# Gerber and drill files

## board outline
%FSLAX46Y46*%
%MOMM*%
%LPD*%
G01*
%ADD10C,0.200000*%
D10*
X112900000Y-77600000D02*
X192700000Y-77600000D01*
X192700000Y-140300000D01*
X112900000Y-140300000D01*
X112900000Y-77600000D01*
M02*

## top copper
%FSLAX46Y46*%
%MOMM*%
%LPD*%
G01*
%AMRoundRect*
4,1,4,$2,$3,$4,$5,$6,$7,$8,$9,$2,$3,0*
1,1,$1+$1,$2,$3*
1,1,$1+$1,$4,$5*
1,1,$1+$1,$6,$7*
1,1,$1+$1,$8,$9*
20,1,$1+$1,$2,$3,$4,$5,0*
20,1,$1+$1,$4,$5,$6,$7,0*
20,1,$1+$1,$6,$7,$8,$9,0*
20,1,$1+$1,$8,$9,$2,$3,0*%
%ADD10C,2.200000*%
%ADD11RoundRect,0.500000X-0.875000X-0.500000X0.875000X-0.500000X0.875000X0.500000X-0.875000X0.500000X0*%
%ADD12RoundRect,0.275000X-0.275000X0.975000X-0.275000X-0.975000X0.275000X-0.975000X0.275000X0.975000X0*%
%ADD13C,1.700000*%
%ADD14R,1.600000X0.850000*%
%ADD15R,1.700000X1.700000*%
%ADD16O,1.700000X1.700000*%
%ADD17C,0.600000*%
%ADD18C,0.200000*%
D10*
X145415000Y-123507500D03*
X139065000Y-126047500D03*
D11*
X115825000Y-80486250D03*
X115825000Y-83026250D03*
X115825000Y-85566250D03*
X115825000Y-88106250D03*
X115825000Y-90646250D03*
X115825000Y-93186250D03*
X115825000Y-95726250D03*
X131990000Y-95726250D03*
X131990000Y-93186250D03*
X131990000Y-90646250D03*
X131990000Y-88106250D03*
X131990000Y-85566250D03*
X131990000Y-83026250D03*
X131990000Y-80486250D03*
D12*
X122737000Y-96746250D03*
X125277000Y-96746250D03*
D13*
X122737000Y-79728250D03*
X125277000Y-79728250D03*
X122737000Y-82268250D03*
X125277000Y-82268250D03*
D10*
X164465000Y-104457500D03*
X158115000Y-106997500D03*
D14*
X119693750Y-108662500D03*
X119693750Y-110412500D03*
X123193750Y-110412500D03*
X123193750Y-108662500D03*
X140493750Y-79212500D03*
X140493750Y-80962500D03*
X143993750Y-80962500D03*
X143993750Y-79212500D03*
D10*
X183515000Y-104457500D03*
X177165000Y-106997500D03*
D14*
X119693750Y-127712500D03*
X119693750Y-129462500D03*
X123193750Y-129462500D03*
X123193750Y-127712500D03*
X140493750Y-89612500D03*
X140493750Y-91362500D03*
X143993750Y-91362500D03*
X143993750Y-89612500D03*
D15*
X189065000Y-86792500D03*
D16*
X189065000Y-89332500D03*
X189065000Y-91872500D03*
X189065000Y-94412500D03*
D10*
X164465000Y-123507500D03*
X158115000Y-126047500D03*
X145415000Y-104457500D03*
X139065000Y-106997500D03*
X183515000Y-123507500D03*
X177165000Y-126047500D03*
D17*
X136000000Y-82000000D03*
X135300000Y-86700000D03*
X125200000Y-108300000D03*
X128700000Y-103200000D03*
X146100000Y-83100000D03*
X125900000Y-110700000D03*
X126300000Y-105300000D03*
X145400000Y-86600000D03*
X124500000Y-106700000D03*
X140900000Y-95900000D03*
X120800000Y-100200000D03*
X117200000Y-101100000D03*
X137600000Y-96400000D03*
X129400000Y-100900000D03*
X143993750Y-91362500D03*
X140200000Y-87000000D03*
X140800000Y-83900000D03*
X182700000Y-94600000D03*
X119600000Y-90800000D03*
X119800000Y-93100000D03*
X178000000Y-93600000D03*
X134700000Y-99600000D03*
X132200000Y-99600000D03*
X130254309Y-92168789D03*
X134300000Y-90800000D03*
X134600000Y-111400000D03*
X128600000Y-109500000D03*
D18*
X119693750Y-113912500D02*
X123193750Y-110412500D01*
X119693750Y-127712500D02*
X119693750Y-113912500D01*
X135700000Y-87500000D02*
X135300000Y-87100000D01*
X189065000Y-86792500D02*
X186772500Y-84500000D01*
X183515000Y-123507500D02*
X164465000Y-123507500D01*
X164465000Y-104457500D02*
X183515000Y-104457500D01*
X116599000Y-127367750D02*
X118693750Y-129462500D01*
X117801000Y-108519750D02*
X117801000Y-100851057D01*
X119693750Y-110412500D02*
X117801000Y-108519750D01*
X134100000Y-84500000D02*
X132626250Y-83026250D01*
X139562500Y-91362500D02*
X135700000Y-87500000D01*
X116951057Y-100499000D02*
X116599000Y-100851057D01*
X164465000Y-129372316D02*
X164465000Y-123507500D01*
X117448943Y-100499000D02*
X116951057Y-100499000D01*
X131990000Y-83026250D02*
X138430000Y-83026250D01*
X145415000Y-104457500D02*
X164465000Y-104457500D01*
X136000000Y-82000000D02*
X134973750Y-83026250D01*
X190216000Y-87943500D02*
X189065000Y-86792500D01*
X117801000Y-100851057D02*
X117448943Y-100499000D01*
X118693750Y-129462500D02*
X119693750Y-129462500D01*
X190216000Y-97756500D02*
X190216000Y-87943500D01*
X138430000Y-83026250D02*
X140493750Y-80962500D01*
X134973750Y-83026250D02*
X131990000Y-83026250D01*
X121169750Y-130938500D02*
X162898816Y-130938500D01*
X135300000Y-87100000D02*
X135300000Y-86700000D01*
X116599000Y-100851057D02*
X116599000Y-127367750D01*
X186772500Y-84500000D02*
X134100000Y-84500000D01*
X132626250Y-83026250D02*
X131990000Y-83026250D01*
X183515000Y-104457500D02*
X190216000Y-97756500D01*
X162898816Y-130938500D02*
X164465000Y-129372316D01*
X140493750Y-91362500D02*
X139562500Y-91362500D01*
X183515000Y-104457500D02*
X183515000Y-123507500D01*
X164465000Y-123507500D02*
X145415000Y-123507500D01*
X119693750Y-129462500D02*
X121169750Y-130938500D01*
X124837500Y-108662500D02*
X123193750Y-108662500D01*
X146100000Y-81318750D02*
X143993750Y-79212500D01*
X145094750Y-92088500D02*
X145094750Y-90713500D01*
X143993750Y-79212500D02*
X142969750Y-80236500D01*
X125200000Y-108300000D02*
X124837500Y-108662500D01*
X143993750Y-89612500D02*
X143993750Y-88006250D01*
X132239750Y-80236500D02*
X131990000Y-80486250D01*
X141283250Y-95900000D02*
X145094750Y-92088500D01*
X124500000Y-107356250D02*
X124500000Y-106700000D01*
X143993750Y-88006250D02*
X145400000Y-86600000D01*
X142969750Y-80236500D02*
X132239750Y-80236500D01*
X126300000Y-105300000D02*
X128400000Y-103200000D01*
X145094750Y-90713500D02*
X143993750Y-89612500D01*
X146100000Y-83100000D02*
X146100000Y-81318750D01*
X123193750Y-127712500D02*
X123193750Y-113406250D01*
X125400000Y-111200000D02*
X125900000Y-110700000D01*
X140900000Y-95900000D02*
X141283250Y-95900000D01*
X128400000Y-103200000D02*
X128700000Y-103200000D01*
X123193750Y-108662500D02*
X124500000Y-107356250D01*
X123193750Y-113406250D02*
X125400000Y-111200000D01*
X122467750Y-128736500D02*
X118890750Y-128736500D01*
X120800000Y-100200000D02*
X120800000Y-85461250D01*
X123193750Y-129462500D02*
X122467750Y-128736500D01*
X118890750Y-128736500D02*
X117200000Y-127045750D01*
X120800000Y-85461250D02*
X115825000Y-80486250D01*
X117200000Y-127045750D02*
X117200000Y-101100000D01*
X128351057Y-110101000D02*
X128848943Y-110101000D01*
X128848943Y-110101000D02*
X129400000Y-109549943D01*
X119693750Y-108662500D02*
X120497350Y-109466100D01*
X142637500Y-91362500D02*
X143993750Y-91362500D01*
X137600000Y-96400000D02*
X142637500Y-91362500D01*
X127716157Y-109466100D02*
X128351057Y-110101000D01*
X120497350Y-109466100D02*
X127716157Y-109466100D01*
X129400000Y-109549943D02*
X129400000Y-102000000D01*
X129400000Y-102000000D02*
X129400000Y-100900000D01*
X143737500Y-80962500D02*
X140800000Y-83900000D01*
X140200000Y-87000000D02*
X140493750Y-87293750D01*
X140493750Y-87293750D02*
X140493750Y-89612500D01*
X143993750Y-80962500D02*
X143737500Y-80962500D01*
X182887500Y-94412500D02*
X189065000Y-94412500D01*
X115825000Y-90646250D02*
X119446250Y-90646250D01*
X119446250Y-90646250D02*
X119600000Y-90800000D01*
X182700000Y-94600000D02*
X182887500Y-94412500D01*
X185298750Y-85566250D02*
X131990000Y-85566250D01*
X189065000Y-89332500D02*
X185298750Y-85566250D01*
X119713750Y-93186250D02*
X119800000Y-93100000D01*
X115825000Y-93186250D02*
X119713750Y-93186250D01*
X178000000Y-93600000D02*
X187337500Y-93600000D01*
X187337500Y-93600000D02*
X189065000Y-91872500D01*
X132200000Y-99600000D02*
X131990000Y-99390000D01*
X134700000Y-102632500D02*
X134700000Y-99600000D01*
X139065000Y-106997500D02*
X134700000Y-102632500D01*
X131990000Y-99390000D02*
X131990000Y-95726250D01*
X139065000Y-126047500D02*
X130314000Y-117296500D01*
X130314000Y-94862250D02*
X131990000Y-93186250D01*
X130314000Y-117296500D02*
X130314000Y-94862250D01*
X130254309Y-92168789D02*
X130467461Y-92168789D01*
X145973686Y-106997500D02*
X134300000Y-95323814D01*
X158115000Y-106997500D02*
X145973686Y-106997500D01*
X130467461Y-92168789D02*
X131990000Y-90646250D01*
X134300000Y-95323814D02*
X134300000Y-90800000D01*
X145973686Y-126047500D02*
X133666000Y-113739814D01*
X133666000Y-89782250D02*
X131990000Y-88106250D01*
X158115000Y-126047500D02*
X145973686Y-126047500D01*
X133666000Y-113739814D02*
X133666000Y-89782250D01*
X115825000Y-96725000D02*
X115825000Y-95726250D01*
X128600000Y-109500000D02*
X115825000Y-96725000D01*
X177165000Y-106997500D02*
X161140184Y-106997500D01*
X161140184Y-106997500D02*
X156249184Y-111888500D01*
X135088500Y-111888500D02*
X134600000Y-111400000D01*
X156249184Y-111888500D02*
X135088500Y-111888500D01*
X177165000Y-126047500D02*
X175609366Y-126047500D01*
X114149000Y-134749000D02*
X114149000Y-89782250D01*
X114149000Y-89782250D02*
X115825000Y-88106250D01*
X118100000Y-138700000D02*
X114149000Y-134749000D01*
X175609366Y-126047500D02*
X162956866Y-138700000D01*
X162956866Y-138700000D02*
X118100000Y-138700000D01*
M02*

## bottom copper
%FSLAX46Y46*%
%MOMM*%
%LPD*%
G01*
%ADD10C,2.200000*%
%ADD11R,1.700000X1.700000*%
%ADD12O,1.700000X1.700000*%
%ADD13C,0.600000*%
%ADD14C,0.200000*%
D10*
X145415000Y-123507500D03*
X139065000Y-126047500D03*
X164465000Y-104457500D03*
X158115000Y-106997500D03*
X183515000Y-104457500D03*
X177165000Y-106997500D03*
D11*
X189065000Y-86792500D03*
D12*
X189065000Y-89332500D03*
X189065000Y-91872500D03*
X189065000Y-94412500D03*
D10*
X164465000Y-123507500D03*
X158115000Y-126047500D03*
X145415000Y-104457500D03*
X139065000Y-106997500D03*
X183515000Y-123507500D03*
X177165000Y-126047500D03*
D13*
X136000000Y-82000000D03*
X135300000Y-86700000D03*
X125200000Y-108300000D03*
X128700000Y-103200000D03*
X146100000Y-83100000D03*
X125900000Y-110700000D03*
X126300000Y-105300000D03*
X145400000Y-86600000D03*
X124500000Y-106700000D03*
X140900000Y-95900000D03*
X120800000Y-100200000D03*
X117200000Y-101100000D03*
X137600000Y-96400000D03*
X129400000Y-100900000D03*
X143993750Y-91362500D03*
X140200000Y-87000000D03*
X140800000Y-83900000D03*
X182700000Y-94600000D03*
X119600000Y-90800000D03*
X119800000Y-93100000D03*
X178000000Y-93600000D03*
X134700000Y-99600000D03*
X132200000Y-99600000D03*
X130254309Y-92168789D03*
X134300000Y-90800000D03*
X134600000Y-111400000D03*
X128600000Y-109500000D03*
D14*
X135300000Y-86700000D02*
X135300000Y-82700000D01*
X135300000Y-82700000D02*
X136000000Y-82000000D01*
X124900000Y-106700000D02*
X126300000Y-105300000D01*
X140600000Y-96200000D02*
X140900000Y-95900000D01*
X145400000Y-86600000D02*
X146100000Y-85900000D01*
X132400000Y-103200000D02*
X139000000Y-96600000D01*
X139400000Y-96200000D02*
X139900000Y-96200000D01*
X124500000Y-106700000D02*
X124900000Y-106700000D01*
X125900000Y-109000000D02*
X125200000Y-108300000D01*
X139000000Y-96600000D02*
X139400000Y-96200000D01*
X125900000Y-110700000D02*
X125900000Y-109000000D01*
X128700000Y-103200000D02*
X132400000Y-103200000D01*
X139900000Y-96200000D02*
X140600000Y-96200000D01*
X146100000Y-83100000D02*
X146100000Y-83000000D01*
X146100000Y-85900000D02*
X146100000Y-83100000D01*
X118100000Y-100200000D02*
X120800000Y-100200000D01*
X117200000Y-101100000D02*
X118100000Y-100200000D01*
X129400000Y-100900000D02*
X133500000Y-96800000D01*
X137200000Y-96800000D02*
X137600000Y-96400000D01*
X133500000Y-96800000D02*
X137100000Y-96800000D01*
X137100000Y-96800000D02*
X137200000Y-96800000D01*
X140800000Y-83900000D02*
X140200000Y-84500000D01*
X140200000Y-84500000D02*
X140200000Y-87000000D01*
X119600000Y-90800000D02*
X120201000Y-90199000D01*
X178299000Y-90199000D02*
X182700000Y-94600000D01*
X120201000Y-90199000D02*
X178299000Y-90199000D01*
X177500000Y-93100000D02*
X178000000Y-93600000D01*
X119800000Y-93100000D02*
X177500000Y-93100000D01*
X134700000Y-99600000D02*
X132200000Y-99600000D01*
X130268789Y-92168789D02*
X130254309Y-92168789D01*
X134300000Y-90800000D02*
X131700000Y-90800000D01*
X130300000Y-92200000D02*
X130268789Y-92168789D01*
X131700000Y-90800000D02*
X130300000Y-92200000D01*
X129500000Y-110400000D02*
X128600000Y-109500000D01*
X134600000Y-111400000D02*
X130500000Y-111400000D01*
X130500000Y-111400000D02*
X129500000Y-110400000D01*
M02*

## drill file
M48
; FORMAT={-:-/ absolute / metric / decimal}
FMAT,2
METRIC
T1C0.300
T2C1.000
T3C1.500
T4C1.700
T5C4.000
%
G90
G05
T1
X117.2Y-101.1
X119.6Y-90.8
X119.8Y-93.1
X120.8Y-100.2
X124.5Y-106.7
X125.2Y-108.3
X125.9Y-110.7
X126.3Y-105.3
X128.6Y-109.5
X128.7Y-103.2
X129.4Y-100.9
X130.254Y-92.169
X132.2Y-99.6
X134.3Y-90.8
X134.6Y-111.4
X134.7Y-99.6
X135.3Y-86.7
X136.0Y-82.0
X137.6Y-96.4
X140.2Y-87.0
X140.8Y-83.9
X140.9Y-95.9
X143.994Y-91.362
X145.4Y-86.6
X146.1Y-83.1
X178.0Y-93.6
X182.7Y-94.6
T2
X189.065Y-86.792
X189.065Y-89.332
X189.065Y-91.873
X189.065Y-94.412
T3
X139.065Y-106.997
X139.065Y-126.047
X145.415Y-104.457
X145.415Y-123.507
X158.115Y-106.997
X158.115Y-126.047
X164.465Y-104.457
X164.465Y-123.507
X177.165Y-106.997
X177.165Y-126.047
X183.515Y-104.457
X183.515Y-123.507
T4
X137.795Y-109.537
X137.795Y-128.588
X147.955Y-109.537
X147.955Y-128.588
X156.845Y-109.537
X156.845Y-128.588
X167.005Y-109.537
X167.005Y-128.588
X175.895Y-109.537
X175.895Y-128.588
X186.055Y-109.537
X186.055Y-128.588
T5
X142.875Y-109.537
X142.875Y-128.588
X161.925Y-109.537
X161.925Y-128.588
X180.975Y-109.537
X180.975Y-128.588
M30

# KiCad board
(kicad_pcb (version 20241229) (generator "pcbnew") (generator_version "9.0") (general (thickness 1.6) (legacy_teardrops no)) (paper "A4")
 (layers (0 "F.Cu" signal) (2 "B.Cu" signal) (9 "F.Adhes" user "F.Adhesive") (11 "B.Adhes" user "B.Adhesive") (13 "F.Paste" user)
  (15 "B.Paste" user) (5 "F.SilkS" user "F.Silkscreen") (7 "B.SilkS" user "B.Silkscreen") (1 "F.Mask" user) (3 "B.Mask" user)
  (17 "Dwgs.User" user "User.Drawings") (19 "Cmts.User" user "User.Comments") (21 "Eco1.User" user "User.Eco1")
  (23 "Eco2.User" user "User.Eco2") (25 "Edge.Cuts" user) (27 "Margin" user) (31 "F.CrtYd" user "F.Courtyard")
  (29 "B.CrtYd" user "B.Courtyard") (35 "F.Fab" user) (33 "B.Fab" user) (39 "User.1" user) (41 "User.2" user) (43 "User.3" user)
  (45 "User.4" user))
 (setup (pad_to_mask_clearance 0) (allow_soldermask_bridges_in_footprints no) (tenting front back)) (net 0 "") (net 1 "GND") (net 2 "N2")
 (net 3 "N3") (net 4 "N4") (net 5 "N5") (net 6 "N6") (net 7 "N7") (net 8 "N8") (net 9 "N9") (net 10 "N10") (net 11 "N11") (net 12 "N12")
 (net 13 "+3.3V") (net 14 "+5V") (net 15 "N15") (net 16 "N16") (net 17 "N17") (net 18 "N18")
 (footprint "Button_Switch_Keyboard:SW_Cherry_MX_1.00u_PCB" (layer "F.Cu") (at 145.415 123.5075)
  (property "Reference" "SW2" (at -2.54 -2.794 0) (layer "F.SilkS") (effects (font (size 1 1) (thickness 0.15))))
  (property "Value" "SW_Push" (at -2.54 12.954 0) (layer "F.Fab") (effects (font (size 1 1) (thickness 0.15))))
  (pad "" np_thru_hole circle (at -7.62 5.08) (size 1.7 1.7) (drill 1.7) (layers "*.Cu" "*.Mask"))
  (pad "" np_thru_hole circle (at -2.54 5.08) (size 4 4) (drill 4) (layers "*.Cu" "*.Mask"))
  (pad "" np_thru_hole circle (at 2.54 5.08) (size 1.7 1.7) (drill 1.7) (layers "*.Cu" "*.Mask"))
  (pad "1" thru_hole circle (at 0 0) (size 2.2 2.2) (drill 1.5) (layers "*.Cu" "*.Mask") (remove_unused_layers no) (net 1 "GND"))
  (pad "2" thru_hole circle (at -6.35 2.54) (size 2.2 2.2) (drill 1.5) (layers "*.Cu" "*.Mask") (remove_unused_layers no) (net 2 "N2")))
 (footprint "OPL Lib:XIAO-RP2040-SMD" (layer "F.Cu") (at 123.825 88.10625)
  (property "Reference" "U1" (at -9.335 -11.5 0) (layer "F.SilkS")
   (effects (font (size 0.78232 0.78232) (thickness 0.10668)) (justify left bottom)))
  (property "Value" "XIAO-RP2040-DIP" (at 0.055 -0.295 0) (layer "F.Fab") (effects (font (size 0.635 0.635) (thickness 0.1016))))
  (pad "1" smd roundrect (at -8 -7.62) (size 2.75 2) (layers "F.Cu" "F.Mask" "F.Paste") (roundrect_rratio 0.25) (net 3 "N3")
   (solder_mask_margin 0.0508) (thermal_bridge_angle 45))
  (pad "2" smd roundrect (at -8 -5.08) (size 2.75 2) (layers "F.Cu" "F.Mask" "F.Paste") (roundrect_rratio 0.25) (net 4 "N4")
   (solder_mask_margin 0.0508) (thermal_bridge_angle 45))
  (pad "3" smd roundrect (at -8 -2.54) (size 2.75 2) (layers "F.Cu" "F.Mask" "F.Paste") (roundrect_rratio 0.25) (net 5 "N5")
   (solder_mask_margin 0.0508) (thermal_bridge_angle 45))
  (pad "4" smd roundrect (at -8 0) (size 2.75 2) (layers "F.Cu" "F.Mask" "F.Paste") (roundrect_rratio 0.25) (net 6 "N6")
   (solder_mask_margin 0.0508) (thermal_bridge_angle 45))
  (pad "5" smd roundrect (at -8 2.54) (size 2.75 2) (layers "F.Cu" "F.Mask" "F.Paste") (roundrect_rratio 0.25) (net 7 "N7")
   (solder_mask_margin 0.0508) (thermal_bridge_angle 45))
  (pad "6" smd roundrect (at -8 5.08) (size 2.75 2) (layers "F.Cu" "F.Mask" "F.Paste") (roundrect_rratio 0.25) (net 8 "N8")
   (solder_mask_margin 0.0508) (thermal_bridge_angle 45))
  (pad "7" smd roundrect (at -8 7.62) (size 2.75 2) (layers "F.Cu" "F.Mask" "F.Paste") (roundrect_rratio 0.25) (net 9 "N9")
   (solder_mask_margin 0.0508) (thermal_bridge_angle 45))
  (pad "8" smd roundrect (at 8.165 7.62) (size 2.75 2) (layers "F.Cu" "F.Mask" "F.Paste") (roundrect_rratio 0.25) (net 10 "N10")
   (solder_mask_margin 0.0508) (thermal_bridge_angle 45))
  (pad "9" smd roundrect (at 8.165 5.08) (size 2.75 2) (layers "F.Cu" "F.Mask" "F.Paste") (roundrect_rratio 0.25) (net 2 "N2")
   (solder_mask_margin 0.0508) (thermal_bridge_angle 45))
  (pad "10" smd roundrect (at 8.165 2.54) (size 2.75 2) (layers "F.Cu" "F.Mask" "F.Paste") (roundrect_rratio 0.25) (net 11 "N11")
   (solder_mask_margin 0.0508) (thermal_bridge_angle 45))
  (pad "11" smd roundrect (at 8.165 0) (size 2.75 2) (layers "F.Cu" "F.Mask" "F.Paste") (roundrect_rratio 0.25) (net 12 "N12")
   (solder_mask_margin 0.0508) (thermal_bridge_angle 45))
  (pad "12" smd roundrect (at 8.165 -2.54) (size 2.75 2) (layers "F.Cu" "F.Mask" "F.Paste") (roundrect_rratio 0.25) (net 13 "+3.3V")
   (solder_mask_margin 0.0508) (thermal_bridge_angle 45))
  (pad "13" smd roundrect (at 8.165 -5.08) (size 2.75 2) (layers "F.Cu" "F.Mask" "F.Paste") (roundrect_rratio 0.25) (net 1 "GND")
   (solder_mask_margin 0.0508) (thermal_bridge_angle 45))
  (pad "14" smd roundrect (at 8.165 -7.62) (size 2.75 2) (layers "F.Cu" "F.Mask" "F.Paste") (roundrect_rratio 0.25) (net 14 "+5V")
   (solder_mask_margin 0.0508) (thermal_bridge_angle 45))
  (pad "15" smd roundrect (at -1.088 8.64 270) (size 2.5 1.1) (layers "F.Cu" "F.Mask" "F.Paste") (roundrect_rratio 0.25)
   (thermal_bridge_angle 45))
  (pad "16" smd roundrect (at 1.452 8.64 270) (size 2.5 1.1) (layers "F.Cu" "F.Mask" "F.Paste") (roundrect_rratio 0.25)
   (thermal_bridge_angle 45))
  (pad "17" smd circle (at -1.088 -8.378) (size 1.7 1.7) (layers "F.Cu" "F.Mask" "F.Paste"))
  (pad "18" smd circle (at 1.452 -8.378) (size 1.7 1.7) (layers "F.Cu" "F.Mask" "F.Paste"))
  (pad "19" smd circle (at -1.088 -5.838) (size 1.7 1.7) (layers "F.Cu" "F.Mask" "F.Paste"))
  (pad "20" smd circle (at 1.452 -5.838) (size 1.7 1.7) (layers "F.Cu" "F.Mask" "F.Paste")))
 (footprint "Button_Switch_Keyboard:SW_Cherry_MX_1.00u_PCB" (layer "F.Cu") (at 164.465 104.4575)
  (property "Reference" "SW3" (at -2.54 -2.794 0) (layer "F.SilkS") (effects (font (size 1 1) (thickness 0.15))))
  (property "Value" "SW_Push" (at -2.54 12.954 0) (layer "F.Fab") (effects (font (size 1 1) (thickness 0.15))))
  (pad "" np_thru_hole circle (at -7.62 5.08) (size 1.7 1.7) (drill 1.7) (layers "*.Cu" "*.Mask"))
  (pad "" np_thru_hole circle (at -2.54 5.08) (size 4 4) (drill 4) (layers "*.Cu" "*.Mask"))
  (pad "" np_thru_hole circle (at 2.54 5.08) (size 1.7 1.7) (drill 1.7) (layers "*.Cu" "*.Mask"))
  (pad "1" thru_hole circle (at 0 0) (size 2.2 2.2) (drill 1.5) (layers "*.Cu" "*.Mask") (remove_unused_layers no) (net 1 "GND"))
  (pad "2" thru_hole circle (at -6.35 2.54) (size 2.2 2.2) (drill 1.5) (layers "*.Cu" "*.Mask") (remove_unused_layers no) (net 11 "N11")))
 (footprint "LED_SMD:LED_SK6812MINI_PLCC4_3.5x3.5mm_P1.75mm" (layer "F.Cu") (at 121.44375 109.5375)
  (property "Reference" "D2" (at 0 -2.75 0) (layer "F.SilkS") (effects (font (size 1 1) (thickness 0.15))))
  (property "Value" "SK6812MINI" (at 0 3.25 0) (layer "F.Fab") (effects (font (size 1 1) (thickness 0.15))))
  (pad "1" smd rect (at -1.75 -0.875) (size 1.6 0.85) (layers "F.Cu" "F.Mask" "F.Paste") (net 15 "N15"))
  (pad "2" smd rect (at -1.75 0.875) (size 1.6 0.85) (layers "F.Cu" "F.Mask" "F.Paste") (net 1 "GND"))
  (pad "3" smd rect (at 1.75 0.875) (size 1.6 0.85) (layers "F.Cu" "F.Mask" "F.Paste") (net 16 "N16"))
  (pad "4" smd rect (at 1.75 -0.875) (size 1.6 0.85) (layers "F.Cu" "F.Mask" "F.Paste") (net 14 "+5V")))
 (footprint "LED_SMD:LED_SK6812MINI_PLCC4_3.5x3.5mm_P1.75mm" (layer "F.Cu") (at 142.24375 80.0875)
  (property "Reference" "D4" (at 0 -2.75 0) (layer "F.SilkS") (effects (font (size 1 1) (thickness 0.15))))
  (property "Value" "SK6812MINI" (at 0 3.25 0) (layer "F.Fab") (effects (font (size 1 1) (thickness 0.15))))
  (pad "1" smd rect (at -1.75 -0.875) (size 1.6 0.85) (layers "F.Cu" "F.Mask" "F.Paste") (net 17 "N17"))
  (pad "2" smd rect (at -1.75 0.875) (size 1.6 0.85) (layers "F.Cu" "F.Mask" "F.Paste") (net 1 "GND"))
  (pad "3" smd rect (at 1.75 0.875) (size 1.6 0.85) (layers "F.Cu" "F.Mask" "F.Paste") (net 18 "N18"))
  (pad "4" smd rect (at 1.75 -0.875) (size 1.6 0.85) (layers "F.Cu" "F.Mask" "F.Paste") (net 14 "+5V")))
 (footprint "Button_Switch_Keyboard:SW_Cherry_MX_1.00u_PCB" (layer "F.Cu") (at 183.515 104.4575)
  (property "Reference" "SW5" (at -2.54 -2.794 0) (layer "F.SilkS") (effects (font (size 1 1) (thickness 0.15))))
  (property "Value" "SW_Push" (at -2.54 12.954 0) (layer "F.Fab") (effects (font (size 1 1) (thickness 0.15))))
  (pad "" np_thru_hole circle (at -7.62 5.08) (size 1.7 1.7) (drill 1.7) (layers "*.Cu" "*.Mask"))
  (pad "" np_thru_hole circle (at -2.54 5.08) (size 4 4) (drill 4) (layers "*.Cu" "*.Mask"))
  (pad "" np_thru_hole circle (at 2.54 5.08) (size 1.7 1.7) (drill 1.7) (layers "*.Cu" "*.Mask"))
  (pad "1" thru_hole circle (at 0 0) (size 2.2 2.2) (drill 1.5) (layers "*.Cu" "*.Mask") (remove_unused_layers no) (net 1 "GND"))
  (pad "2" thru_hole circle (at -6.35 2.54) (size 2.2 2.2) (drill 1.5) (layers "*.Cu" "*.Mask") (remove_unused_layers no) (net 9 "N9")))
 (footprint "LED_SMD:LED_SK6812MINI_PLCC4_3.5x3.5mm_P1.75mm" (layer "F.Cu") (at 121.44375 128.5875)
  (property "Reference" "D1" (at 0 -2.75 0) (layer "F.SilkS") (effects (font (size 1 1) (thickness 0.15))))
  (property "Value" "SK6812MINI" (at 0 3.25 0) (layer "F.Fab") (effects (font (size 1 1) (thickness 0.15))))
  (pad "1" smd rect (at -1.75 -0.875) (size 1.6 0.85) (layers "F.Cu" "F.Mask" "F.Paste") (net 16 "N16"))
  (pad "2" smd rect (at -1.75 0.875) (size 1.6 0.85) (layers "F.Cu" "F.Mask" "F.Paste") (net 1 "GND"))
  (pad "3" smd rect (at 1.75 0.875) (size 1.6 0.85) (layers "F.Cu" "F.Mask" "F.Paste") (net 3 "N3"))
  (pad "4" smd rect (at 1.75 -0.875) (size 1.6 0.85) (layers "F.Cu" "F.Mask" "F.Paste") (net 14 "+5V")))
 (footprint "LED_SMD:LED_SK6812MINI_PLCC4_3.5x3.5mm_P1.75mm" (layer "F.Cu") (at 142.24375 90.4875)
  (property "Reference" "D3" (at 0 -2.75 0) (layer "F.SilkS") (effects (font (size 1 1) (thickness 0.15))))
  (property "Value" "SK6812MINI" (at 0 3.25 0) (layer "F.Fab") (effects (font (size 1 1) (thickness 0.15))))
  (pad "1" smd rect (at -1.75 -0.875) (size 1.6 0.85) (layers "F.Cu" "F.Mask" "F.Paste") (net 18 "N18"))
  (pad "2" smd rect (at -1.75 0.875) (size 1.6 0.85) (layers "F.Cu" "F.Mask" "F.Paste") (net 1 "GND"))
  (pad "3" smd rect (at 1.75 0.875) (size 1.6 0.85) (layers "F.Cu" "F.Mask" "F.Paste") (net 15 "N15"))
  (pad "4" smd rect (at 1.75 -0.875) (size 1.6 0.85) (layers "F.Cu" "F.Mask" "F.Paste") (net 14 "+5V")))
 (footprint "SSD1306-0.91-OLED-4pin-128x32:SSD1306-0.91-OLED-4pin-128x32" (layer "F.Cu") (at 152.565 84.6025)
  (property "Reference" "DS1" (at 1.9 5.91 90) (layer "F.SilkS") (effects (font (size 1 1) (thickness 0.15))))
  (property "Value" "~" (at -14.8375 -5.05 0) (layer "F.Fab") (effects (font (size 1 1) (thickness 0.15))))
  (pad "1" thru_hole rect (at 36.5 2.19) (size 1.7 1.7) (drill 1) (layers "*.Cu" "*.Mask") (remove_unused_layers no) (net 1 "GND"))
  (pad "2" thru_hole oval (at 36.5 4.73) (size 1.7 1.7) (drill 1) (layers "*.Cu" "*.Mask") (remove_unused_layers no) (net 13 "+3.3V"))
  (pad "3" thru_hole oval (at 36.5 7.27) (size 1.7 1.7) (drill 1) (layers "*.Cu" "*.Mask") (remove_unused_layers no) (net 8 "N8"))
  (pad "4" thru_hole oval (at 36.5 9.81) (size 1.7 1.7) (drill 1) (layers "*.Cu" "*.Mask") (remove_unused_layers no) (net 7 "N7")))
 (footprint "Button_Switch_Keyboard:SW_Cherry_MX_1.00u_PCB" (layer "F.Cu") (at 164.465 123.5075)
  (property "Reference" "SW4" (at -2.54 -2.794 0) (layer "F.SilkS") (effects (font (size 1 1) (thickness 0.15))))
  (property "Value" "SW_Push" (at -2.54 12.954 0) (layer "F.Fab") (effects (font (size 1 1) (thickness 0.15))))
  (pad "" np_thru_hole circle (at -7.62 5.08) (size 1.7 1.7) (drill 1.7) (layers "*.Cu" "*.Mask"))
  (pad "" np_thru_hole circle (at -2.54 5.08) (size 4 4) (drill 4) (layers "*.Cu" "*.Mask"))
  (pad "" np_thru_hole circle (at 2.54 5.08) (size 1.7 1.7) (drill 1.7) (layers "*.Cu" "*.Mask"))
  (pad "1" thru_hole circle (at 0 0) (size 2.2 2.2) (drill 1.5) (layers "*.Cu" "*.Mask") (remove_unused_layers no) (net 1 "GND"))
  (pad "2" thru_hole circle (at -6.35 2.54) (size 2.2 2.2) (drill 1.5) (layers "*.Cu" "*.Mask") (remove_unused_layers no) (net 12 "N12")))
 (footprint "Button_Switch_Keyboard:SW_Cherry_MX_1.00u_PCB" (layer "F.Cu") (at 145.415 104.4575)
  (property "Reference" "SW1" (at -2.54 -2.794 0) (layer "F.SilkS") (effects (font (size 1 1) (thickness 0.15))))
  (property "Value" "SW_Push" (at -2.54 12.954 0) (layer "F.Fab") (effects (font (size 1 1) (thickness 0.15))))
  (pad "" np_thru_hole circle (at -7.62 5.08) (size 1.7 1.7) (drill 1.7) (layers "*.Cu" "*.Mask"))
  (pad "" np_thru_hole circle (at -2.54 5.08) (size 4 4) (drill 4) (layers "*.Cu" "*.Mask"))
  (pad "" np_thru_hole circle (at 2.54 5.08) (size 1.7 1.7) (drill 1.7) (layers "*.Cu" "*.Mask"))
  (pad "1" thru_hole circle (at 0 0) (size 2.2 2.2) (drill 1.5) (layers "*.Cu" "*.Mask") (remove_unused_layers no) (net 1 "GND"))
  (pad "2" thru_hole circle (at -6.35 2.54) (size 2.2 2.2) (drill 1.5) (layers "*.Cu" "*.Mask") (remove_unused_layers no) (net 10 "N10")))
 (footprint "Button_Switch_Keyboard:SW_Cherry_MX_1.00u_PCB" (layer "F.Cu") (at 183.515 123.5075)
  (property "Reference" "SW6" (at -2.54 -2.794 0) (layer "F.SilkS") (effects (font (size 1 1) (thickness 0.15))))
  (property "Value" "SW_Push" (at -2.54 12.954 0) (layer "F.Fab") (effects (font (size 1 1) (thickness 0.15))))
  (pad "" np_thru_hole circle (at -7.62 5.08) (size 1.7 1.7) (drill 1.7) (layers "*.Cu" "*.Mask"))
  (pad "" np_thru_hole circle (at -2.54 5.08) (size 4 4) (drill 4) (layers "*.Cu" "*.Mask"))
  (pad "" np_thru_hole circle (at 2.54 5.08) (size 1.7 1.7) (drill 1.7) (layers "*.Cu" "*.Mask"))
  (pad "1" thru_hole circle (at 0 0) (size 2.2 2.2) (drill 1.5) (layers "*.Cu" "*.Mask") (remove_unused_layers no) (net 1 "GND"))
  (pad "2" thru_hole circle (at -6.35 2.54) (size 2.2 2.2) (drill 1.5) (layers "*.Cu" "*.Mask") (remove_unused_layers no) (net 6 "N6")))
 (gr_rect (start 112.9 77.6) (end 192.7 140.3) (stroke (width 0.2) (type solid)) (fill no) (layer "Edge.Cuts"))
 (segment (start 119.69375 113.9125) (end 123.19375 110.4125) (width 0.2) (layer "F.Cu") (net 16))
 (segment (start 119.69375 127.7125) (end 119.69375 113.9125) (width 0.2) (layer "F.Cu") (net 16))
 (segment (start 135.7 87.5) (end 135.3 87.1) (width 0.2) (layer "F.Cu") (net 1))
 (segment (start 189.065 86.7925) (end 186.7725 84.5) (width 0.2) (layer "F.Cu") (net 1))
 (segment (start 183.515 123.5075) (end 164.465 123.5075) (width 0.2) (layer "F.Cu") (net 1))
 (segment (start 164.465 104.4575) (end 183.515 104.4575) (width 0.2) (layer "F.Cu") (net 1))
 (segment (start 116.599 127.36775) (end 118.69375 129.4625) (width 0.2) (layer "F.Cu") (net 1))
 (segment (start 117.801 108.51975) (end 117.801 100.851057) (width 0.2) (layer "F.Cu") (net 1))
 (segment (start 119.69375 110.4125) (end 117.801 108.51975) (width 0.2) (layer "F.Cu") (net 1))
 (segment (start 134.1 84.5) (end 132.62625 83.02625) (width 0.2) (layer "F.Cu") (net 1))
 (segment (start 139.5625 91.3625) (end 135.7 87.5) (width 0.2) (layer "F.Cu") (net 1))
 (segment (start 116.951057 100.499) (end 116.599 100.851057) (width 0.2) (layer "F.Cu") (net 1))
 (segment (start 164.465 129.372316) (end 164.465 123.5075) (width 0.2) (layer "F.Cu") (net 1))
 (segment (start 117.448943 100.499) (end 116.951057 100.499) (width 0.2) (layer "F.Cu") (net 1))
 (segment (start 131.99 83.02625) (end 138.43 83.02625) (width 0.2) (layer "F.Cu") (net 1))
 (segment (start 145.415 104.4575) (end 164.465 104.4575) (width 0.2) (layer "F.Cu") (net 1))
 (segment (start 136 82) (end 134.97375 83.02625) (width 0.2) (layer "F.Cu") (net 1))
 (segment (start 190.216 87.9435) (end 189.065 86.7925) (width 0.2) (layer "F.Cu") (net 1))
 (segment (start 117.801 100.851057) (end 117.448943 100.499) (width 0.2) (layer "F.Cu") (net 1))
 (segment (start 118.69375 129.4625) (end 119.69375 129.4625) (width 0.2) (layer "F.Cu") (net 1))
 (segment (start 190.216 97.7565) (end 190.216 87.9435) (width 0.2) (layer "F.Cu") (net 1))
 (segment (start 138.43 83.02625) (end 140.49375 80.9625) (width 0.2) (layer "F.Cu") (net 1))
 (segment (start 134.97375 83.02625) (end 131.99 83.02625) (width 0.2) (layer "F.Cu") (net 1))
 (segment (start 121.16975 130.9385) (end 162.898816 130.9385) (width 0.2) (layer "F.Cu") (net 1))
 (segment (start 135.3 87.1) (end 135.3 86.7) (width 0.2) (layer "F.Cu") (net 1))
 (segment (start 116.599 100.851057) (end 116.599 127.36775) (width 0.2) (layer "F.Cu") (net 1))
 (segment (start 186.7725 84.5) (end 134.1 84.5) (width 0.2) (layer "F.Cu") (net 1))
 (segment (start 132.62625 83.02625) (end 131.99 83.02625) (width 0.2) (layer "F.Cu") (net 1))
 (segment (start 183.515 104.4575) (end 190.216 97.7565) (width 0.2) (layer "F.Cu") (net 1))
 (segment (start 162.898816 130.9385) (end 164.465 129.372316) (width 0.2) (layer "F.Cu") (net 1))
 (segment (start 140.49375 91.3625) (end 139.5625 91.3625) (width 0.2) (layer "F.Cu") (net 1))
 (segment (start 183.515 104.4575) (end 183.515 123.5075) (width 0.2) (layer "F.Cu") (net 1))
 (segment (start 164.465 123.5075) (end 145.415 123.5075) (width 0.2) (layer "F.Cu") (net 1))
 (segment (start 119.69375 129.4625) (end 121.16975 130.9385) (width 0.2) (layer "F.Cu") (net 1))
 (via (at 136 82) (size 0.6) (drill 0.3) (layers "F.Cu" "B.Cu") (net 1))
 (via (at 135.3 86.7) (size 0.6) (drill 0.3) (layers "F.Cu" "B.Cu") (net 1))
 (segment (start 135.3 86.7) (end 135.3 82.7) (width 0.2) (layer "B.Cu") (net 1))
 (segment (start 135.3 82.7) (end 136 82) (width 0.2) (layer "B.Cu") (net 1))
 (segment (start 124.8375 108.6625) (end 123.19375 108.6625) (width 0.2) (layer "F.Cu") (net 14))
 (segment (start 146.1 81.31875) (end 143.99375 79.2125) (width 0.2) (layer "F.Cu") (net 14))
 (segment (start 145.09475 92.0885) (end 145.09475 90.7135) (width 0.2) (layer "F.Cu") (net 14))
 (segment (start 143.99375 79.2125) (end 142.96975 80.2365) (width 0.2) (layer "F.Cu") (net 14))
 (segment (start 125.2 108.3) (end 124.8375 108.6625) (width 0.2) (layer "F.Cu") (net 14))
 (segment (start 143.99375 89.6125) (end 143.99375 88.00625) (width 0.2) (layer "F.Cu") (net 14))
 (segment (start 132.23975 80.2365) (end 131.99 80.48625) (width 0.2) (layer "F.Cu") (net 14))
 (segment (start 141.28325 95.9) (end 145.09475 92.0885) (width 0.2) (layer "F.Cu") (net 14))
 (segment (start 124.5 107.35625) (end 124.5 106.7) (width 0.2) (layer "F.Cu") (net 14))
 (segment (start 143.99375 88.00625) (end 145.4 86.6) (width 0.2) (layer "F.Cu") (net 14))
 (segment (start 142.96975 80.2365) (end 132.23975 80.2365) (width 0.2) (layer "F.Cu") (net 14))
 (segment (start 126.3 105.3) (end 128.4 103.2) (width 0.2) (layer "F.Cu") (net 14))
 (segment (start 145.09475 90.7135) (end 143.99375 89.6125) (width 0.2) (layer "F.Cu") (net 14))
 (segment (start 146.1 83.1) (end 146.1 81.31875) (width 0.2) (layer "F.Cu") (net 14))
 (segment (start 123.19375 127.7125) (end 123.19375 113.40625) (width 0.2) (layer "F.Cu") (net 14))
 (segment (start 125.4 111.2) (end 125.9 110.7) (width 0.2) (layer "F.Cu") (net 14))
 (segment (start 140.9 95.9) (end 141.28325 95.9) (width 0.2) (layer "F.Cu") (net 14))
 (segment (start 128.4 103.2) (end 128.7 103.2) (width 0.2) (layer "F.Cu") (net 14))
 (segment (start 123.19375 108.6625) (end 124.5 107.35625) (width 0.2) (layer "F.Cu") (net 14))
 (segment (start 123.19375 113.40625) (end 125.4 111.2) (width 0.2) (layer "F.Cu") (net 14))
 (via (at 125.2 108.3) (size 0.6) (drill 0.3) (layers "F.Cu" "B.Cu") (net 14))
 (via (at 128.7 103.2) (size 0.6) (drill 0.3) (layers "F.Cu" "B.Cu") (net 14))
 (via (at 146.1 83.1) (size 0.6) (drill 0.3) (layers "F.Cu" "B.Cu") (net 14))
 (via (at 125.9 110.7) (size 0.6) (drill 0.3) (layers "F.Cu" "B.Cu") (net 14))
 (via (at 126.3 105.3) (size 0.6) (drill 0.3) (layers "F.Cu" "B.Cu") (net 14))
 (via (at 145.4 86.6) (size 0.6) (drill 0.3) (layers "F.Cu" "B.Cu") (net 14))
 (via (at 124.5 106.7) (size 0.6) (drill 0.3) (layers "F.Cu" "B.Cu") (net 14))
 (via (at 140.9 95.9) (size 0.6) (drill 0.3) (layers "F.Cu" "B.Cu") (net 14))
 (segment (start 124.9 106.7) (end 126.3 105.3) (width 0.2) (layer "B.Cu") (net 14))
 (segment (start 140.6 96.2) (end 140.9 95.9) (width 0.2) (layer "B.Cu") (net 14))
 (segment (start 145.4 86.6) (end 146.1 85.9) (width 0.2) (layer "B.Cu") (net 14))
 (segment (start 132.4 103.2) (end 139 96.6) (width 0.2) (layer "B.Cu") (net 14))
 (segment (start 139.4 96.2) (end 139.9 96.2) (width 0.2) (layer "B.Cu") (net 14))
 (segment (start 124.5 106.7) (end 124.9 106.7) (width 0.2) (layer "B.Cu") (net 14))
 (segment (start 125.9 109) (end 125.2 108.3) (width 0.2) (layer "B.Cu") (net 14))
 (segment (start 139 96.6) (end 139.4 96.2) (width 0.2) (layer "B.Cu") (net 14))
 (segment (start 125.9 110.7) (end 125.9 109) (width 0.2) (layer "B.Cu") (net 14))
 (segment (start 128.7 103.2) (end 132.4 103.2) (width 0.2) (layer "B.Cu") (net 14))
 (segment (start 139.9 96.2) (end 140.6 96.2) (width 0.2) (layer "B.Cu") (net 14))
 (segment (start 146.1 83.1) (end 146.1 83) (width 0.2) (layer "B.Cu") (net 14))
 (segment (start 146.1 85.9) (end 146.1 83.1) (width 0.2) (layer "B.Cu") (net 14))
 (segment (start 122.46775 128.7365) (end 118.89075 128.7365) (width 0.2) (layer "F.Cu") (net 3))
 (segment (start 120.8 100.2) (end 120.8 85.46125) (width 0.2) (layer "F.Cu") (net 3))
 (segment (start 123.19375 129.4625) (end 122.46775 128.7365) (width 0.2) (layer "F.Cu") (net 3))
 (segment (start 118.89075 128.7365) (end 117.2 127.04575) (width 0.2) (layer "F.Cu") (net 3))
 (segment (start 120.8 85.46125) (end 115.825 80.48625) (width 0.2) (layer "F.Cu") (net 3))
 (segment (start 117.2 127.04575) (end 117.2 101.1) (width 0.2) (layer "F.Cu") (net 3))
 (via (at 120.8 100.2) (size 0.6) (drill 0.3) (layers "F.Cu" "B.Cu") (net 3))
 (via (at 117.2 101.1) (size 0.6) (drill 0.3) (layers "F.Cu" "B.Cu") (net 3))
 (segment (start 118.1 100.2) (end 120.8 100.2) (width 0.2) (layer "B.Cu") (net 3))
 (segment (start 117.2 101.1) (end 118.1 100.2) (width 0.2) (layer "B.Cu") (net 3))
 (segment (start 128.351057 110.101) (end 128.848943 110.101) (width 0.2) (layer "F.Cu") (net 15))
 (segment (start 128.848943 110.101) (end 129.4 109.549943) (width 0.2) (layer "F.Cu") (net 15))
 (segment (start 119.69375 108.6625) (end 120.49735 109.4661) (width 0.2) (layer "F.Cu") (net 15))
 (segment (start 142.6375 91.3625) (end 143.99375 91.3625) (width 0.2) (layer "F.Cu") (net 15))
 (segment (start 137.6 96.4) (end 142.6375 91.3625) (width 0.2) (layer "F.Cu") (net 15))
 (segment (start 127.716157 109.4661) (end 128.351057 110.101) (width 0.2) (layer "F.Cu") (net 15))
 (segment (start 120.49735 109.4661) (end 127.716157 109.4661) (width 0.2) (layer "F.Cu") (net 15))
 (segment (start 129.4 109.549943) (end 129.4 102) (width 0.2) (layer "F.Cu") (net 15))
 (segment (start 129.4 102) (end 129.4 100.9) (width 0.2) (layer "F.Cu") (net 15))
 (via (at 137.6 96.4) (size 0.6) (drill 0.3) (layers "F.Cu" "B.Cu") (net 15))
 (via (at 129.4 100.9) (size 0.6) (drill 0.3) (layers "F.Cu" "B.Cu") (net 15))
 (via (at 143.99375 91.3625) (size 0.6) (drill 0.3) (layers "F.Cu" "B.Cu") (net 15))
 (segment (start 129.4 100.9) (end 133.5 96.8) (width 0.2) (layer "B.Cu") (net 15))
 (segment (start 137.2 96.8) (end 137.6 96.4) (width 0.2) (layer "B.Cu") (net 15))
 (segment (start 133.5 96.8) (end 137.1 96.8) (width 0.2) (layer "B.Cu") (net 15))
 (segment (start 137.1 96.8) (end 137.2 96.8) (width 0.2) (layer "B.Cu") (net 15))
 (segment (start 143.7375 80.9625) (end 140.8 83.9) (width 0.2) (layer "F.Cu") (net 18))
 (segment (start 140.2 87) (end 140.49375 87.29375) (width 0.2) (layer "F.Cu") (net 18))
 (segment (start 140.49375 87.29375) (end 140.49375 89.6125) (width 0.2) (layer "F.Cu") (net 18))
 (segment (start 143.99375 80.9625) (end 143.7375 80.9625) (width 0.2) (layer "F.Cu") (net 18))
 (via (at 140.2 87) (size 0.6) (drill 0.3) (layers "F.Cu" "B.Cu") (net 18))
 (via (at 140.8 83.9) (size 0.6) (drill 0.3) (layers "F.Cu" "B.Cu") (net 18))
 (segment (start 140.8 83.9) (end 140.2 84.5) (width 0.2) (layer "B.Cu") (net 18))
 (segment (start 140.2 84.5) (end 140.2 87) (width 0.2) (layer "B.Cu") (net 18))
 (segment (start 182.8875 94.4125) (end 189.065 94.4125) (width 0.2) (layer "F.Cu") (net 7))
 (segment (start 115.825 90.64625) (end 119.44625 90.64625) (width 0.2) (layer "F.Cu") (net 7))
 (segment (start 119.44625 90.64625) (end 119.6 90.8) (width 0.2) (layer "F.Cu") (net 7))
 (segment (start 182.7 94.6) (end 182.8875 94.4125) (width 0.2) (layer "F.Cu") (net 7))
 (via (at 182.7 94.6) (size 0.6) (drill 0.3) (layers "F.Cu" "B.Cu") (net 7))
 (via (at 119.6 90.8) (size 0.6) (drill 0.3) (layers "F.Cu" "B.Cu") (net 7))
 (segment (start 119.6 90.8) (end 120.201 90.199) (width 0.2) (layer "B.Cu") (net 7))
 (segment (start 178.299 90.199) (end 182.7 94.6) (width 0.2) (layer "B.Cu") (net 7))
 (segment (start 120.201 90.199) (end 178.299 90.199) (width 0.2) (layer "B.Cu") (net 7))
 (segment (start 185.29875 85.56625) (end 131.99 85.56625) (width 0.2) (layer "F.Cu") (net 13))
 (segment (start 189.065 89.3325) (end 185.29875 85.56625) (width 0.2) (layer "F.Cu") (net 13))
 (segment (start 119.71375 93.18625) (end 119.8 93.1) (width 0.2) (layer "F.Cu") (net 8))
 (segment (start 115.825 93.18625) (end 119.71375 93.18625) (width 0.2) (layer "F.Cu") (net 8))
 (segment (start 178 93.6) (end 187.3375 93.6) (width 0.2) (layer "F.Cu") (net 8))
 (segment (start 187.3375 93.6) (end 189.065 91.8725) (width 0.2) (layer "F.Cu") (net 8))
 (via (at 119.8 93.1) (size 0.6) (drill 0.3) (layers "F.Cu" "B.Cu") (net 8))
 (via (at 178 93.6) (size 0.6) (drill 0.3) (layers "F.Cu" "B.Cu") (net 8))
 (segment (start 177.5 93.1) (end 178 93.6) (width 0.2) (layer "B.Cu") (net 8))
 (segment (start 119.8 93.1) (end 177.5 93.1) (width 0.2) (layer "B.Cu") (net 8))
 (segment (start 132.2 99.6) (end 131.99 99.39) (width 0.2) (layer "F.Cu") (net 10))
 (segment (start 134.7 102.6325) (end 134.7 99.6) (width 0.2) (layer "F.Cu") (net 10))
 (segment (start 139.065 106.9975) (end 134.7 102.6325) (width 0.2) (layer "F.Cu") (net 10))
 (segment (start 131.99 99.39) (end 131.99 95.72625) (width 0.2) (layer "F.Cu") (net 10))
 (via (at 134.7 99.6) (size 0.6) (drill 0.3) (layers "F.Cu" "B.Cu") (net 10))
 (via (at 132.2 99.6) (size 0.6) (drill 0.3) (layers "F.Cu" "B.Cu") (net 10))
 (segment (start 134.7 99.6) (end 132.2 99.6) (width 0.2) (layer "B.Cu") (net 10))
 (segment (start 139.065 126.0475) (end 130.314 117.2965) (width 0.2) (layer "F.Cu") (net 2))
 (segment (start 130.314 94.86225) (end 131.99 93.18625) (width 0.2) (layer "F.Cu") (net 2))
 (segment (start 130.314 117.2965) (end 130.314 94.86225) (width 0.2) (layer "F.Cu") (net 2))
 (segment (start 130.254309 92.168789) (end 130.467461 92.168789) (width 0.2) (layer "F.Cu") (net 11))
 (segment (start 145.973686 106.9975) (end 134.3 95.323814) (width 0.2) (layer "F.Cu") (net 11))
 (segment (start 158.115 106.9975) (end 145.973686 106.9975) (width 0.2) (layer "F.Cu") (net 11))
 (segment (start 130.467461 92.168789) (end 131.99 90.64625) (width 0.2) (layer "F.Cu") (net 11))
 (segment (start 134.3 95.323814) (end 134.3 90.8) (width 0.2) (layer "F.Cu") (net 11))
 (via (at 130.254309 92.168789) (size 0.6) (drill 0.3) (layers "F.Cu" "B.Cu") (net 11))
 (via (at 134.3 90.8) (size 0.6) (drill 0.3) (layers "F.Cu" "B.Cu") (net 11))
 (segment (start 130.268789 92.168789) (end 130.254309 92.168789) (width 0.2) (layer "B.Cu") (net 11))
 (segment (start 134.3 90.8) (end 131.7 90.8) (width 0.2) (layer "B.Cu") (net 11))
 (segment (start 130.3 92.2) (end 130.268789 92.168789) (width 0.2) (layer "B.Cu") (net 11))
 (segment (start 131.7 90.8) (end 130.3 92.2) (width 0.2) (layer "B.Cu") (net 11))
 (segment (start 145.973686 126.0475) (end 133.666 113.739814) (width 0.2) (layer "F.Cu") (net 12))
 (segment (start 133.666 89.78225) (end 131.99 88.10625) (width 0.2) (layer "F.Cu") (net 12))
 (segment (start 158.115 126.0475) (end 145.973686 126.0475) (width 0.2) (layer "F.Cu") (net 12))
 (segment (start 133.666 113.739814) (end 133.666 89.78225) (width 0.2) (layer "F.Cu") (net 12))
 (segment (start 115.825 96.725) (end 115.825 95.72625) (width 0.2) (layer "F.Cu") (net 9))
 (segment (start 128.6 109.5) (end 115.825 96.725) (width 0.2) (layer "F.Cu") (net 9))
 (segment (start 177.165 106.9975) (end 161.140184 106.9975) (width 0.2) (layer "F.Cu") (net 9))
 (segment (start 161.140184 106.9975) (end 156.249184 111.8885) (width 0.2) (layer "F.Cu") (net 9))
 (segment (start 135.0885 111.8885) (end 134.6 111.4) (width 0.2) (layer "F.Cu") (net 9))
 (segment (start 156.249184 111.8885) (end 135.0885 111.8885) (width 0.2) (layer "F.Cu") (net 9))
 (via (at 134.6 111.4) (size 0.6) (drill 0.3) (layers "F.Cu" "B.Cu") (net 9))
 (via (at 128.6 109.5) (size 0.6) (drill 0.3) (layers "F.Cu" "B.Cu") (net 9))
 (segment (start 129.5 110.4) (end 128.6 109.5) (width 0.2) (layer "B.Cu") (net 9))
 (segment (start 134.6 111.4) (end 130.5 111.4) (width 0.2) (layer "B.Cu") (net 9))
 (segment (start 130.5 111.4) (end 129.5 110.4) (width 0.2) (layer "B.Cu") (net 9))
 (segment (start 177.165 126.0475) (end 175.609366 126.0475) (width 0.2) (layer "F.Cu") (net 6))
 (segment (start 114.149 134.749) (end 114.149 89.78225) (width 0.2) (layer "F.Cu") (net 6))
 (segment (start 114.149 89.78225) (end 115.825 88.10625) (width 0.2) (layer "F.Cu") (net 6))
 (segment (start 118.1 138.7) (end 114.149 134.749) (width 0.2) (layer "F.Cu") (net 6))
 (segment (start 175.609366 126.0475) (end 162.956866 138.7) (width 0.2) (layer "F.Cu") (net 6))
 (segment (start 162.956866 138.7) (end 118.1 138.7) (width 0.2) (layer "F.Cu") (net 6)))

